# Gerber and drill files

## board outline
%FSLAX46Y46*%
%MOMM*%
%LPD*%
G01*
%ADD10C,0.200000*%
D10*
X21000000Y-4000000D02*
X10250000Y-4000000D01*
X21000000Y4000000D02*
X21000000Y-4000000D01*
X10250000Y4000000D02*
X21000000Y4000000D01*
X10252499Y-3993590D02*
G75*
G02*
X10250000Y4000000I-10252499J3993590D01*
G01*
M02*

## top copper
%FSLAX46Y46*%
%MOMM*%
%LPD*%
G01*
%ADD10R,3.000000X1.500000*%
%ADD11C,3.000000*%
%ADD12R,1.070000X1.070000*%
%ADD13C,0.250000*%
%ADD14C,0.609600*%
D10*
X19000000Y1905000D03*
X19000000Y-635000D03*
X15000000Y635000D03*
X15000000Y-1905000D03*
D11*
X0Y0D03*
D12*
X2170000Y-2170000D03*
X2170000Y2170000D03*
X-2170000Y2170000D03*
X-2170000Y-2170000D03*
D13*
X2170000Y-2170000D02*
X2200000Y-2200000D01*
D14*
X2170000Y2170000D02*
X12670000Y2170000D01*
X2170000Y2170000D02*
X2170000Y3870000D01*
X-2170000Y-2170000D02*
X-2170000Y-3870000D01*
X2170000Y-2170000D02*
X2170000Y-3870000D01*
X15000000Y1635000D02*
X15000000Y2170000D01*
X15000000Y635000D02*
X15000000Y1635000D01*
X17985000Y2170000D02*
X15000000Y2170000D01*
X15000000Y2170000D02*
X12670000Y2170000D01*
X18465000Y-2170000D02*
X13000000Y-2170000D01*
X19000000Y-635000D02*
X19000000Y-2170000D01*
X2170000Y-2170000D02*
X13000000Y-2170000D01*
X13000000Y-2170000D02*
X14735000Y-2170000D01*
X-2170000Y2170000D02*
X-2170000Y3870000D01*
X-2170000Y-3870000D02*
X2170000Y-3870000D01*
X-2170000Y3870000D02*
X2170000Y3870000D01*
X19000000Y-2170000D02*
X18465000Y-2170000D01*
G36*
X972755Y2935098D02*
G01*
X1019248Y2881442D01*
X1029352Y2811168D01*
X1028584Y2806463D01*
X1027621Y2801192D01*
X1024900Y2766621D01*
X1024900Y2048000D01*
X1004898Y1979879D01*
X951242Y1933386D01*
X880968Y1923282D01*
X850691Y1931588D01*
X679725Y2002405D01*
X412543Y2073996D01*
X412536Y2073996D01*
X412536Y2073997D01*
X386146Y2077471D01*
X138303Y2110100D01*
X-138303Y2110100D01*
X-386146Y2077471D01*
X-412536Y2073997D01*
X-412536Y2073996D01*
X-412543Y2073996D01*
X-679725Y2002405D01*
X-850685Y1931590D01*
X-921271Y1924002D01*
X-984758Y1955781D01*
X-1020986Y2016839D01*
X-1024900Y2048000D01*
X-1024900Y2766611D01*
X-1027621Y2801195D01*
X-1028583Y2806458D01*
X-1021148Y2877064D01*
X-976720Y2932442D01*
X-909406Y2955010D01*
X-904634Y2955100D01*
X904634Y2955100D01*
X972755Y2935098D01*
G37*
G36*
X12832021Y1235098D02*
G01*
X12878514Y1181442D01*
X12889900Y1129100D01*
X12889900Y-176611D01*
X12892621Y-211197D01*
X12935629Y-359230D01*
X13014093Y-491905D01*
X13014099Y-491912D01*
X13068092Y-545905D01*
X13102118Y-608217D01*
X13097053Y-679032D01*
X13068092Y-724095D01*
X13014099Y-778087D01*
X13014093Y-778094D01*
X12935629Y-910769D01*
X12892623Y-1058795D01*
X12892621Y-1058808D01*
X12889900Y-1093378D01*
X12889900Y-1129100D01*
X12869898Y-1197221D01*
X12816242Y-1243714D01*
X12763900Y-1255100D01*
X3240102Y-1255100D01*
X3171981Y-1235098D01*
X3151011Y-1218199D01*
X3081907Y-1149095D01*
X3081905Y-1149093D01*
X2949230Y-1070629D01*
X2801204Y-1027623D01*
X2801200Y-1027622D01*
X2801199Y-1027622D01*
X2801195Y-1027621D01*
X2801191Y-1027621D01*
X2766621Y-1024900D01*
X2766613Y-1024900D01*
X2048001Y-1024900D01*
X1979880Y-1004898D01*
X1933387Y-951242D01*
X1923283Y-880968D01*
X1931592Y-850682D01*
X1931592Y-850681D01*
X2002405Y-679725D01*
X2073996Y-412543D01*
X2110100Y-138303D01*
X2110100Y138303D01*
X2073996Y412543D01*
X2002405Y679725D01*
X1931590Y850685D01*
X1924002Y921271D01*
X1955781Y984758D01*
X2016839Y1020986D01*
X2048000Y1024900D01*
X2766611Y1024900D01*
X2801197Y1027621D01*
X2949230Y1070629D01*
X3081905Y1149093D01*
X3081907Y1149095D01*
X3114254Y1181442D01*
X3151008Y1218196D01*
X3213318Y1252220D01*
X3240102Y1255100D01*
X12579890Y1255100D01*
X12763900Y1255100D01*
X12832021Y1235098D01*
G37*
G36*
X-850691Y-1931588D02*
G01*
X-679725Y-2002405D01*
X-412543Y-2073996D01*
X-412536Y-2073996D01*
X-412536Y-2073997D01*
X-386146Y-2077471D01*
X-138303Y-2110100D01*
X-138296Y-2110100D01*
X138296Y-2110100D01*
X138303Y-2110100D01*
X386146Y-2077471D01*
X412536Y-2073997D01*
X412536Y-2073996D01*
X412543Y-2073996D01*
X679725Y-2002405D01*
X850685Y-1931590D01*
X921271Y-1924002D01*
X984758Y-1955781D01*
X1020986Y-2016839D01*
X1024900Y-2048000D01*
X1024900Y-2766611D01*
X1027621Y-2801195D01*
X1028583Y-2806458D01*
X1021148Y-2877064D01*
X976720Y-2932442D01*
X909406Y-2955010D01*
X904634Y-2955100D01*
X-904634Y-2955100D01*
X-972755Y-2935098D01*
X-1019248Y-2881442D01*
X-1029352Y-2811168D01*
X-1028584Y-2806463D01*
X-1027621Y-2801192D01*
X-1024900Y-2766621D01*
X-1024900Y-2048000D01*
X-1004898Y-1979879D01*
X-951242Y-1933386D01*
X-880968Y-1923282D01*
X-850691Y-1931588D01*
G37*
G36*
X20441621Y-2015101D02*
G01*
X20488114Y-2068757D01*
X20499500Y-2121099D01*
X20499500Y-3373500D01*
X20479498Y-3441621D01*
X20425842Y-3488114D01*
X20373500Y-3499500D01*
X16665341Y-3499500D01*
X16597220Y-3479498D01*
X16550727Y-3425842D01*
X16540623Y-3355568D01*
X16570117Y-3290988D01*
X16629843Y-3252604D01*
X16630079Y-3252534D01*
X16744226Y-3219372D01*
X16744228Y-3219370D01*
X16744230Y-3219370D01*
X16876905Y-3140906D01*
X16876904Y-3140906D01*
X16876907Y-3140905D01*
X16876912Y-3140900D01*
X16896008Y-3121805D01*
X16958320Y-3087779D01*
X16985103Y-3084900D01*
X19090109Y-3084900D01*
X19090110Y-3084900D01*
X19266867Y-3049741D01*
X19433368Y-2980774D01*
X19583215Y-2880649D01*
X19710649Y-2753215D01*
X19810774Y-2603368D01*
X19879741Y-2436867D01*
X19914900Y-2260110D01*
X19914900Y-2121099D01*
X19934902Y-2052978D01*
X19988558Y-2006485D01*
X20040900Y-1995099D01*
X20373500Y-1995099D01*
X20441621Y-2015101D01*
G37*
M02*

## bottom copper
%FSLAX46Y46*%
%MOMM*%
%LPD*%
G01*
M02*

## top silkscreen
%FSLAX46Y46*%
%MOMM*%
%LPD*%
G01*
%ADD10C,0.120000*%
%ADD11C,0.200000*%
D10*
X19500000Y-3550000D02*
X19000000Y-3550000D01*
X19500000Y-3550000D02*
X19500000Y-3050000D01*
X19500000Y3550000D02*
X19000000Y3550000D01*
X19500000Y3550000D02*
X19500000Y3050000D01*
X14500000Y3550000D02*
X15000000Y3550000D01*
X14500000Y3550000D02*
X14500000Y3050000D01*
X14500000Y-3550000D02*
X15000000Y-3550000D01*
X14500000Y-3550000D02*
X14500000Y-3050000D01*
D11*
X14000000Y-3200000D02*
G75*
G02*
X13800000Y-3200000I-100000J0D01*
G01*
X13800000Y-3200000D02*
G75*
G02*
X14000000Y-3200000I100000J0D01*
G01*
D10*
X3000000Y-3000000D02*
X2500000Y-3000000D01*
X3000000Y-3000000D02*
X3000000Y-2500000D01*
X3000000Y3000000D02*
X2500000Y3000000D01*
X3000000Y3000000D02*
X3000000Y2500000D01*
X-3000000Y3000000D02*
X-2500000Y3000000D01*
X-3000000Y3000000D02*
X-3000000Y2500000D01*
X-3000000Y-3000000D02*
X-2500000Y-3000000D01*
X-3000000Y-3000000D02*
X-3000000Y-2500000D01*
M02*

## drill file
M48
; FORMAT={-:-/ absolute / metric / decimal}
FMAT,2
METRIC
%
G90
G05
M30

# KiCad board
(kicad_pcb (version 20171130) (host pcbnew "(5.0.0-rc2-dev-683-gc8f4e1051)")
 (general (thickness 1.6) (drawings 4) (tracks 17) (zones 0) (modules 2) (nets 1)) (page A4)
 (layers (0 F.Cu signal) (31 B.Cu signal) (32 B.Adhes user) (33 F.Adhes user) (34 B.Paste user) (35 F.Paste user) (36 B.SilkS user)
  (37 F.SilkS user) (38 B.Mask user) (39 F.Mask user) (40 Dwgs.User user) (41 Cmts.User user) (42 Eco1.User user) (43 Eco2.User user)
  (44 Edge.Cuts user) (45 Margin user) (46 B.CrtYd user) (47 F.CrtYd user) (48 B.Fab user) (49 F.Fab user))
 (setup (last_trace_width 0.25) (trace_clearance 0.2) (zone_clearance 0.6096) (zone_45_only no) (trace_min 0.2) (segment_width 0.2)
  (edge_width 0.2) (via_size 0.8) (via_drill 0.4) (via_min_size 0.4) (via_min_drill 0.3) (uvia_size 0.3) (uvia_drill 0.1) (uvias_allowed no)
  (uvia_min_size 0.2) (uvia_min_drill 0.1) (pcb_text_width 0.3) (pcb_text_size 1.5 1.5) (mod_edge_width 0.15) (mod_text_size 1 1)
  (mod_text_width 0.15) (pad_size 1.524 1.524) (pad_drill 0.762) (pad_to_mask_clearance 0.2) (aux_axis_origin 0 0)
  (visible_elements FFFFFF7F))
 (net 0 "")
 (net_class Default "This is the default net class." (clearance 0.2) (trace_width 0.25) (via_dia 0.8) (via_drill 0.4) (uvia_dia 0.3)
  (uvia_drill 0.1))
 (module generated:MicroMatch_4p (layer F.Cu) (at 17 0 90)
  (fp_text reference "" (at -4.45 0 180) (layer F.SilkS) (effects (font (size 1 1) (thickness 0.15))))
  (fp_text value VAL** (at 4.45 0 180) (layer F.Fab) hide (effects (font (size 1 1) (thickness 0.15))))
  (fp_line (start -3.55 2.5) (end -3.55 2) (layer F.SilkS) (width 0.12))
  (fp_line (start -3.55 2.5) (end -3.05 2.5) (layer F.SilkS) (width 0.12))
  (fp_line (start 3.55 2.5) (end 3.55 2) (layer F.SilkS) (width 0.12))
  (fp_line (start 3.55 2.5) (end 3.05 2.5) (layer F.SilkS) (width 0.12))
  (fp_line (start 3.55 -2.5) (end 3.55 -2) (layer F.SilkS) (width 0.12))
  (fp_line (start 3.55 -2.5) (end 3.05 -2.5) (layer F.SilkS) (width 0.12))
  (fp_line (start -3.55 -2.5) (end -3.55 -2) (layer F.SilkS) (width 0.12))
  (fp_line (start -3.55 -2.5) (end -3.05 -2.5) (layer F.SilkS) (width 0.12))
  (fp_circle (center -3.2 -3.1) (end -3.1 -3.1) (layer F.SilkS) (width 0.2))
  (pad 4 smd rect (at 1.905 2 90) (size 1.5 3) (layers F.Cu F.Paste F.Mask))
  (pad 2 smd rect (at -0.635 2 90) (size 1.5 3) (layers F.Cu F.Paste F.Mask))
  (pad 3 smd rect (at 0.635 -2 90) (size 1.5 3) (layers F.Cu F.Paste F.Mask))
  (pad 1 smd rect (at -1.905 -2 90) (size 1.5 3) (layers F.Cu F.Paste F.Mask)))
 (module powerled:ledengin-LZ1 (layer F.Cu) (at 0 0 90)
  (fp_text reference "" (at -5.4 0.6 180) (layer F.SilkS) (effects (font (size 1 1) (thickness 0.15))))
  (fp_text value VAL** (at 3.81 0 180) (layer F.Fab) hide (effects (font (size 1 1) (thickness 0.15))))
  (fp_line (start -3 3) (end -3 2.5) (layer F.SilkS) (width 0.12))
  (fp_line (start -3 3) (end -2.5 3) (layer F.SilkS) (width 0.12))
  (fp_line (start 3 3) (end 3 2.5) (layer F.SilkS) (width 0.12))
  (fp_line (start 3 3) (end 2.5 3) (layer F.SilkS) (width 0.12))
  (fp_line (start 3 -3) (end 3 -2.5) (layer F.SilkS) (width 0.12))
  (fp_line (start 3 -3) (end 2.5 -3) (layer F.SilkS) (width 0.12))
  (fp_line (start -3 -3) (end -3 -2.5) (layer F.SilkS) (width 0.12))
  (fp_line (start -3 -3) (end -2.5 -3) (layer F.SilkS) (width 0.12))
  (pad 5 smd circle (at 0 0 90) (size 3 3) (layers F.Cu F.Paste F.Mask))
  (pad 4 smd rect (at -2.17 2.17 90) (size 1.07 1.07) (layers F.Cu F.Paste F.Mask))
  (pad 3 smd rect (at 2.17 2.17 90) (size 1.07 1.07) (layers F.Cu F.Paste F.Mask))
  (pad 2 smd rect (at 2.17 -2.17 90) (size 1.07 1.07) (layers F.Cu F.Paste F.Mask))
  (pad 1 smd rect (at -2.17 -2.17 90) (size 1.07 1.07) (layers F.Cu F.Paste F.Mask)))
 (gr_line (start 21 4) (end 10.25 4) (layer Edge.Cuts) (width 0.2))
 (gr_line (start 21 -4) (end 21 4) (layer Edge.Cuts) (width 0.2))
 (gr_line (start 10.25 -4) (end 21 -4) (layer Edge.Cuts) (width 0.2))
 (gr_arc (start 0 0) (end 10.25 -4) (angle -317.4) (layer Edge.Cuts) (width 0.2))
 (segment (start 2.17 2.17) (end 2.2 2.2) (width 0.25) (layer F.Cu) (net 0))
 (segment (start 2.17 -2.17) (end 12.67 -2.17) (width 0.6096) (layer F.Cu) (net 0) (status 40000))
 (segment (start 2.17 -2.17) (end 2.17 -3.87) (width 0.6096) (layer F.Cu) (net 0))
 (segment (start -2.17 2.17) (end -2.17 3.87) (width 0.6096) (layer F.Cu) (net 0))
 (segment (start 2.17 2.17) (end 2.17 3.87) (width 0.6096) (layer F.Cu) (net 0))
 (segment (start 15 -1.635) (end 15 -2.17) (width 0.6096) (layer F.Cu) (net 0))
 (segment (start 15 -0.635) (end 15 -1.635) (width 0.6096) (layer F.Cu) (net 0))
 (segment (start 17.985 -2.17) (end 15 -2.17) (width 0.6096) (layer F.Cu) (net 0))
 (segment (start 15 -2.17) (end 12.67 -2.17) (width 0.6096) (layer F.Cu) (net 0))
 (segment (start 18.465 2.17) (end 13 2.17) (width 0.6096) (layer F.Cu) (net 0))
 (segment (start 19 0.635) (end 19 2.17) (width 0.6096) (layer F.Cu) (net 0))
 (segment (start 2.17 2.17) (end 13 2.17) (width 0.6096) (layer F.Cu) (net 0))
 (segment (start 13 2.17) (end 14.735 2.17) (width 0.6096) (layer F.Cu) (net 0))
 (segment (start -2.17 -2.17) (end -2.17 -3.87) (width 0.6096) (layer F.Cu) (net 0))
 (segment (start -2.17 3.87) (end 2.17 3.87) (width 0.6096) (layer F.Cu) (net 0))
 (segment (start -2.17 -3.87) (end 2.17 -3.87) (width 0.6096) (layer F.Cu) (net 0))
 (segment (start 19 2.17) (end 18.465 2.17) (width 0.6096) (layer F.Cu) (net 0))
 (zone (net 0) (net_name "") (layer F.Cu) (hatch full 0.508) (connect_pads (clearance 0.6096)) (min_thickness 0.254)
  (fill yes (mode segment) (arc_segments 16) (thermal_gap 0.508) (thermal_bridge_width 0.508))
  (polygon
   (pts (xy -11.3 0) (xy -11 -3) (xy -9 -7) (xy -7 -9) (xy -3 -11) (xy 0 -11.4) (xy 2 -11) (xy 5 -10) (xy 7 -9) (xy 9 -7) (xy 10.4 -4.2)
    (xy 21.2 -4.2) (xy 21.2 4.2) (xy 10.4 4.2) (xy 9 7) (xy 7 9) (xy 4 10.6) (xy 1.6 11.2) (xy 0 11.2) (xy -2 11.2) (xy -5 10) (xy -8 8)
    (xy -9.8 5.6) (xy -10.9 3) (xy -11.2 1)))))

